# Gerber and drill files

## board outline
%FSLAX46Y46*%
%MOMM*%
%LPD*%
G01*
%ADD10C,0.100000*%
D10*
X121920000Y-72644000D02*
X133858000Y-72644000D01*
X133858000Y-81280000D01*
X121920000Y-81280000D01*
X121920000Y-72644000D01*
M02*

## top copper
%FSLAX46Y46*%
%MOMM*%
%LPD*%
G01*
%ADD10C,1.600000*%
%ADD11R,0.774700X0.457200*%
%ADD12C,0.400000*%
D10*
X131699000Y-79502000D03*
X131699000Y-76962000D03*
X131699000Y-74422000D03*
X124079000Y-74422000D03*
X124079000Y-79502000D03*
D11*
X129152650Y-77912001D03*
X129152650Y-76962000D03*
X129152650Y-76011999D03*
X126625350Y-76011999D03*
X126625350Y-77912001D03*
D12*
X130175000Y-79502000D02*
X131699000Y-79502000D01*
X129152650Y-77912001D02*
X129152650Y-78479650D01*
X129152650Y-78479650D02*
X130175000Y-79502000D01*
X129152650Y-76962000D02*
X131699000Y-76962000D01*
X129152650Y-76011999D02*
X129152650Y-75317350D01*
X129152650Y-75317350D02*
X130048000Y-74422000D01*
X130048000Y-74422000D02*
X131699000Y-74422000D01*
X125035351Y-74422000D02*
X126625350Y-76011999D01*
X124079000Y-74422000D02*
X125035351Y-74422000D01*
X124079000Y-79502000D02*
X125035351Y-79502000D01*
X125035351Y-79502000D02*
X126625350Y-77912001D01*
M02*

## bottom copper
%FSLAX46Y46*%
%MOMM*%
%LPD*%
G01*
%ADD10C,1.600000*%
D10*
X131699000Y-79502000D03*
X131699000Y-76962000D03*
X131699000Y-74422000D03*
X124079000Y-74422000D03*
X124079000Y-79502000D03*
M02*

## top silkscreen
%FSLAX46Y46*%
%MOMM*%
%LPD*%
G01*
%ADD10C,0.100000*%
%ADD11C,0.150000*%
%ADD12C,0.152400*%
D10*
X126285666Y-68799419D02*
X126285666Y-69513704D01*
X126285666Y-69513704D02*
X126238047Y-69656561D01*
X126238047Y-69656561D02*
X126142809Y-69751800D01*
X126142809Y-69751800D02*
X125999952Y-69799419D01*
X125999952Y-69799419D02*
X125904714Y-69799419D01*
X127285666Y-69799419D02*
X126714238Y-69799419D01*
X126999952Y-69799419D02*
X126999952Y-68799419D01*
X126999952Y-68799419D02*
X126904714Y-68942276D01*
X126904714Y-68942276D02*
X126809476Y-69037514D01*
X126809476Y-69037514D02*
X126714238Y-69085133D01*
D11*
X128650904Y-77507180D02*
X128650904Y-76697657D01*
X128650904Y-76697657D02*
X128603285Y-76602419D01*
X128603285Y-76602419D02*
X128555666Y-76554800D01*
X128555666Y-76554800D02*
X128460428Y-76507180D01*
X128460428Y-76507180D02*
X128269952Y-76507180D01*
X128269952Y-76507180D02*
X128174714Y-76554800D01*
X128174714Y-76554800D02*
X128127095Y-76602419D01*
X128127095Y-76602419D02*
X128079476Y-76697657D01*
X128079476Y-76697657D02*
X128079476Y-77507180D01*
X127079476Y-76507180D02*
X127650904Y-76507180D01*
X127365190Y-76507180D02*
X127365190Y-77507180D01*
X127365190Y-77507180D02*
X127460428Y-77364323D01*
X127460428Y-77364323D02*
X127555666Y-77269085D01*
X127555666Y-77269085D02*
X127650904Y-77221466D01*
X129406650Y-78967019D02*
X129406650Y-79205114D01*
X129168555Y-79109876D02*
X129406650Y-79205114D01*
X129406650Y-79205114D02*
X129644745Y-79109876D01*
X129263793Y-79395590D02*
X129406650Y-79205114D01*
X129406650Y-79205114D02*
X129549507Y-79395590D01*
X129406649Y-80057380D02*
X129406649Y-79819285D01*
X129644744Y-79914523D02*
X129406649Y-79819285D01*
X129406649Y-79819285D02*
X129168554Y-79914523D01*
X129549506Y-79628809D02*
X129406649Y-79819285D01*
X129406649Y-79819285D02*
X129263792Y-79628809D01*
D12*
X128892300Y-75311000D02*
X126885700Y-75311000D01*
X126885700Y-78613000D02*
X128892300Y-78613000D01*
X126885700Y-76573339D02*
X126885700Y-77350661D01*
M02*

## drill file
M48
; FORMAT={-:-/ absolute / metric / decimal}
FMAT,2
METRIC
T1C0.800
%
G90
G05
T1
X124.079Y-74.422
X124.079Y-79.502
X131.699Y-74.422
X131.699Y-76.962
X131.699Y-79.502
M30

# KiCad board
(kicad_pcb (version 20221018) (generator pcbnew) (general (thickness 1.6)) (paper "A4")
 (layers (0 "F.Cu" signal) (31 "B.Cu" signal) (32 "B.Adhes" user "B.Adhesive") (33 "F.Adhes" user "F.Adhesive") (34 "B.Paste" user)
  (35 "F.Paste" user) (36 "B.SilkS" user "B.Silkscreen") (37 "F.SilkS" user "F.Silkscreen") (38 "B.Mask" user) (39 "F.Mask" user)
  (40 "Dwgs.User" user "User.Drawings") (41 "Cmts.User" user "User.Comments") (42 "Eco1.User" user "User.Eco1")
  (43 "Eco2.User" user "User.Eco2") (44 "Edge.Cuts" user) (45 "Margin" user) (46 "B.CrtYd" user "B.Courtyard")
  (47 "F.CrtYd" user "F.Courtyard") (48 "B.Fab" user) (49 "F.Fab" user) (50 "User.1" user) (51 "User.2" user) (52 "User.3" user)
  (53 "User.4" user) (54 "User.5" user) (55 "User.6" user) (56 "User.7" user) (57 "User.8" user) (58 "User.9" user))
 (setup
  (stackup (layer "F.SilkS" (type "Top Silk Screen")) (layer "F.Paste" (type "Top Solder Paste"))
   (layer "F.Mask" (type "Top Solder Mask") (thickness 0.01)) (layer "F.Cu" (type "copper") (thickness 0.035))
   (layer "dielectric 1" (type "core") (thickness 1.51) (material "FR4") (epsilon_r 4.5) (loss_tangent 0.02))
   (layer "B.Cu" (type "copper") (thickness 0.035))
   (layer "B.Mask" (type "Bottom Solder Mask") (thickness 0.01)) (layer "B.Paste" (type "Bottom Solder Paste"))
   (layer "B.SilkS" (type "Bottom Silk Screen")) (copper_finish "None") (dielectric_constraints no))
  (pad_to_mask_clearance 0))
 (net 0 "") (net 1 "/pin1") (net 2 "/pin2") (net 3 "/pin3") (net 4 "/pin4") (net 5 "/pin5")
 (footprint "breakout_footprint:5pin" (layer "F.Cu") (at 126.619 79.502)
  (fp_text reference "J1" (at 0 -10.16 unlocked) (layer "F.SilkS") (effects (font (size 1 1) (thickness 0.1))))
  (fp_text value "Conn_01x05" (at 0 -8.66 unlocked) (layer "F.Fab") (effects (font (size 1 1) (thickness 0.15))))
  (pad "1" thru_hole circle (at 5.08 0) (size 1.6 1.6) (drill 0.8) (layers "*.Cu" "*.Mask") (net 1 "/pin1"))
  (pad "2" thru_hole circle (at 5.08 -2.54) (size 1.6 1.6) (drill 0.8) (layers "*.Cu" "*.Mask") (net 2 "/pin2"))
  (pad "3" thru_hole circle (at 5.08 -5.08) (size 1.6 1.6) (drill 0.8) (layers "*.Cu" "*.Mask") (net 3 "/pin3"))
  (pad "4" thru_hole circle (at -2.54 -5.08) (size 1.6 1.6) (drill 0.8) (layers "*.Cu" "*.Mask") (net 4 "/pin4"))
  (pad "5" thru_hole circle (at -2.54 0) (size 1.6 1.6) (drill 0.8) (layers "*.Cu" "*.Mask") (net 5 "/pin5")))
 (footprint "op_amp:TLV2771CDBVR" (layer "F.Cu") (at 127.889 76.962 180)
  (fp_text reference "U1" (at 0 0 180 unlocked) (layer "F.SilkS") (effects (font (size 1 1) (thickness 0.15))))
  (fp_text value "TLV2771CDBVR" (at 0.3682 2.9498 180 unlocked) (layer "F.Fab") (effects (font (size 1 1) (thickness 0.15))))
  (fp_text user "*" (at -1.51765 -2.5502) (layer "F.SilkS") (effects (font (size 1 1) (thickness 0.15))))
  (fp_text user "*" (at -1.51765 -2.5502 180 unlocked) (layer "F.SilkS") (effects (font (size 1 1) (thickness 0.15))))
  (fp_line (start -1.0033 1.651) (end 1.0033 1.651) (stroke (width 0.1524) (type solid)) (layer "F.SilkS"))
  (fp_line (start 1.0033 -1.651) (end -1.0033 -1.651) (stroke (width 0.1524) (type solid)) (layer "F.SilkS"))
  (fp_line (start 1.0033 0.388661) (end 1.0033 -0.388661) (stroke (width 0.1524) (type solid)) (layer "F.SilkS"))
  (pad "1" smd rect (at -1.26365 -0.950001 180) (size 0.7747 0.4572) (layers "F.Cu" "F.Paste" "F.Mask") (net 1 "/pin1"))
  (pad "2" smd rect (at -1.26365 0 180) (size 0.7747 0.4572) (layers "F.Cu" "F.Paste" "F.Mask") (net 2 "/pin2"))
  (pad "3" smd rect (at -1.26365 0.950001 180) (size 0.7747 0.4572) (layers "F.Cu" "F.Paste" "F.Mask") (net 3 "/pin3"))
  (pad "4" smd rect (at 1.26365 0.950001 180) (size 0.7747 0.4572) (layers "F.Cu" "F.Paste" "F.Mask") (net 4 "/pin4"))
  (pad "5" smd rect (at 1.26365 -0.950001 180) (size 0.7747 0.4572) (layers "F.Cu" "F.Paste" "F.Mask") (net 5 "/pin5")))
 (gr_rect (start 121.92 72.644) (end 133.858 81.28) (stroke (width 0.1) (type default)) (fill none) (layer "Edge.Cuts"))
 (segment (start 130.175 79.502) (end 131.699 79.502) (width 0.4) (layer "F.Cu") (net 1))
 (segment (start 129.15265 77.912001) (end 129.15265 78.47965) (width 0.4) (layer "F.Cu") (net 1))
 (segment (start 129.15265 78.47965) (end 130.175 79.502) (width 0.4) (layer "F.Cu") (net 1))
 (segment (start 129.15265 76.962) (end 131.699 76.962) (width 0.4) (layer "F.Cu") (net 2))
 (segment (start 129.15265 76.011999) (end 129.15265 75.31735) (width 0.4) (layer "F.Cu") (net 3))
 (segment (start 129.15265 75.31735) (end 130.048 74.422) (width 0.4) (layer "F.Cu") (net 3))
 (segment (start 130.048 74.422) (end 131.699 74.422) (width 0.4) (layer "F.Cu") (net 3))
 (segment (start 125.035351 74.422) (end 126.62535 76.011999) (width 0.4) (layer "F.Cu") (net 4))
 (segment (start 124.079 74.422) (end 125.035351 74.422) (width 0.4) (layer "F.Cu") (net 4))
 (segment (start 124.079 79.502) (end 125.035351 79.502) (width 0.4) (layer "F.Cu") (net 5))
 (segment (start 125.035351 79.502) (end 126.62535 77.912001) (width 0.4) (layer "F.Cu") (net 5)))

